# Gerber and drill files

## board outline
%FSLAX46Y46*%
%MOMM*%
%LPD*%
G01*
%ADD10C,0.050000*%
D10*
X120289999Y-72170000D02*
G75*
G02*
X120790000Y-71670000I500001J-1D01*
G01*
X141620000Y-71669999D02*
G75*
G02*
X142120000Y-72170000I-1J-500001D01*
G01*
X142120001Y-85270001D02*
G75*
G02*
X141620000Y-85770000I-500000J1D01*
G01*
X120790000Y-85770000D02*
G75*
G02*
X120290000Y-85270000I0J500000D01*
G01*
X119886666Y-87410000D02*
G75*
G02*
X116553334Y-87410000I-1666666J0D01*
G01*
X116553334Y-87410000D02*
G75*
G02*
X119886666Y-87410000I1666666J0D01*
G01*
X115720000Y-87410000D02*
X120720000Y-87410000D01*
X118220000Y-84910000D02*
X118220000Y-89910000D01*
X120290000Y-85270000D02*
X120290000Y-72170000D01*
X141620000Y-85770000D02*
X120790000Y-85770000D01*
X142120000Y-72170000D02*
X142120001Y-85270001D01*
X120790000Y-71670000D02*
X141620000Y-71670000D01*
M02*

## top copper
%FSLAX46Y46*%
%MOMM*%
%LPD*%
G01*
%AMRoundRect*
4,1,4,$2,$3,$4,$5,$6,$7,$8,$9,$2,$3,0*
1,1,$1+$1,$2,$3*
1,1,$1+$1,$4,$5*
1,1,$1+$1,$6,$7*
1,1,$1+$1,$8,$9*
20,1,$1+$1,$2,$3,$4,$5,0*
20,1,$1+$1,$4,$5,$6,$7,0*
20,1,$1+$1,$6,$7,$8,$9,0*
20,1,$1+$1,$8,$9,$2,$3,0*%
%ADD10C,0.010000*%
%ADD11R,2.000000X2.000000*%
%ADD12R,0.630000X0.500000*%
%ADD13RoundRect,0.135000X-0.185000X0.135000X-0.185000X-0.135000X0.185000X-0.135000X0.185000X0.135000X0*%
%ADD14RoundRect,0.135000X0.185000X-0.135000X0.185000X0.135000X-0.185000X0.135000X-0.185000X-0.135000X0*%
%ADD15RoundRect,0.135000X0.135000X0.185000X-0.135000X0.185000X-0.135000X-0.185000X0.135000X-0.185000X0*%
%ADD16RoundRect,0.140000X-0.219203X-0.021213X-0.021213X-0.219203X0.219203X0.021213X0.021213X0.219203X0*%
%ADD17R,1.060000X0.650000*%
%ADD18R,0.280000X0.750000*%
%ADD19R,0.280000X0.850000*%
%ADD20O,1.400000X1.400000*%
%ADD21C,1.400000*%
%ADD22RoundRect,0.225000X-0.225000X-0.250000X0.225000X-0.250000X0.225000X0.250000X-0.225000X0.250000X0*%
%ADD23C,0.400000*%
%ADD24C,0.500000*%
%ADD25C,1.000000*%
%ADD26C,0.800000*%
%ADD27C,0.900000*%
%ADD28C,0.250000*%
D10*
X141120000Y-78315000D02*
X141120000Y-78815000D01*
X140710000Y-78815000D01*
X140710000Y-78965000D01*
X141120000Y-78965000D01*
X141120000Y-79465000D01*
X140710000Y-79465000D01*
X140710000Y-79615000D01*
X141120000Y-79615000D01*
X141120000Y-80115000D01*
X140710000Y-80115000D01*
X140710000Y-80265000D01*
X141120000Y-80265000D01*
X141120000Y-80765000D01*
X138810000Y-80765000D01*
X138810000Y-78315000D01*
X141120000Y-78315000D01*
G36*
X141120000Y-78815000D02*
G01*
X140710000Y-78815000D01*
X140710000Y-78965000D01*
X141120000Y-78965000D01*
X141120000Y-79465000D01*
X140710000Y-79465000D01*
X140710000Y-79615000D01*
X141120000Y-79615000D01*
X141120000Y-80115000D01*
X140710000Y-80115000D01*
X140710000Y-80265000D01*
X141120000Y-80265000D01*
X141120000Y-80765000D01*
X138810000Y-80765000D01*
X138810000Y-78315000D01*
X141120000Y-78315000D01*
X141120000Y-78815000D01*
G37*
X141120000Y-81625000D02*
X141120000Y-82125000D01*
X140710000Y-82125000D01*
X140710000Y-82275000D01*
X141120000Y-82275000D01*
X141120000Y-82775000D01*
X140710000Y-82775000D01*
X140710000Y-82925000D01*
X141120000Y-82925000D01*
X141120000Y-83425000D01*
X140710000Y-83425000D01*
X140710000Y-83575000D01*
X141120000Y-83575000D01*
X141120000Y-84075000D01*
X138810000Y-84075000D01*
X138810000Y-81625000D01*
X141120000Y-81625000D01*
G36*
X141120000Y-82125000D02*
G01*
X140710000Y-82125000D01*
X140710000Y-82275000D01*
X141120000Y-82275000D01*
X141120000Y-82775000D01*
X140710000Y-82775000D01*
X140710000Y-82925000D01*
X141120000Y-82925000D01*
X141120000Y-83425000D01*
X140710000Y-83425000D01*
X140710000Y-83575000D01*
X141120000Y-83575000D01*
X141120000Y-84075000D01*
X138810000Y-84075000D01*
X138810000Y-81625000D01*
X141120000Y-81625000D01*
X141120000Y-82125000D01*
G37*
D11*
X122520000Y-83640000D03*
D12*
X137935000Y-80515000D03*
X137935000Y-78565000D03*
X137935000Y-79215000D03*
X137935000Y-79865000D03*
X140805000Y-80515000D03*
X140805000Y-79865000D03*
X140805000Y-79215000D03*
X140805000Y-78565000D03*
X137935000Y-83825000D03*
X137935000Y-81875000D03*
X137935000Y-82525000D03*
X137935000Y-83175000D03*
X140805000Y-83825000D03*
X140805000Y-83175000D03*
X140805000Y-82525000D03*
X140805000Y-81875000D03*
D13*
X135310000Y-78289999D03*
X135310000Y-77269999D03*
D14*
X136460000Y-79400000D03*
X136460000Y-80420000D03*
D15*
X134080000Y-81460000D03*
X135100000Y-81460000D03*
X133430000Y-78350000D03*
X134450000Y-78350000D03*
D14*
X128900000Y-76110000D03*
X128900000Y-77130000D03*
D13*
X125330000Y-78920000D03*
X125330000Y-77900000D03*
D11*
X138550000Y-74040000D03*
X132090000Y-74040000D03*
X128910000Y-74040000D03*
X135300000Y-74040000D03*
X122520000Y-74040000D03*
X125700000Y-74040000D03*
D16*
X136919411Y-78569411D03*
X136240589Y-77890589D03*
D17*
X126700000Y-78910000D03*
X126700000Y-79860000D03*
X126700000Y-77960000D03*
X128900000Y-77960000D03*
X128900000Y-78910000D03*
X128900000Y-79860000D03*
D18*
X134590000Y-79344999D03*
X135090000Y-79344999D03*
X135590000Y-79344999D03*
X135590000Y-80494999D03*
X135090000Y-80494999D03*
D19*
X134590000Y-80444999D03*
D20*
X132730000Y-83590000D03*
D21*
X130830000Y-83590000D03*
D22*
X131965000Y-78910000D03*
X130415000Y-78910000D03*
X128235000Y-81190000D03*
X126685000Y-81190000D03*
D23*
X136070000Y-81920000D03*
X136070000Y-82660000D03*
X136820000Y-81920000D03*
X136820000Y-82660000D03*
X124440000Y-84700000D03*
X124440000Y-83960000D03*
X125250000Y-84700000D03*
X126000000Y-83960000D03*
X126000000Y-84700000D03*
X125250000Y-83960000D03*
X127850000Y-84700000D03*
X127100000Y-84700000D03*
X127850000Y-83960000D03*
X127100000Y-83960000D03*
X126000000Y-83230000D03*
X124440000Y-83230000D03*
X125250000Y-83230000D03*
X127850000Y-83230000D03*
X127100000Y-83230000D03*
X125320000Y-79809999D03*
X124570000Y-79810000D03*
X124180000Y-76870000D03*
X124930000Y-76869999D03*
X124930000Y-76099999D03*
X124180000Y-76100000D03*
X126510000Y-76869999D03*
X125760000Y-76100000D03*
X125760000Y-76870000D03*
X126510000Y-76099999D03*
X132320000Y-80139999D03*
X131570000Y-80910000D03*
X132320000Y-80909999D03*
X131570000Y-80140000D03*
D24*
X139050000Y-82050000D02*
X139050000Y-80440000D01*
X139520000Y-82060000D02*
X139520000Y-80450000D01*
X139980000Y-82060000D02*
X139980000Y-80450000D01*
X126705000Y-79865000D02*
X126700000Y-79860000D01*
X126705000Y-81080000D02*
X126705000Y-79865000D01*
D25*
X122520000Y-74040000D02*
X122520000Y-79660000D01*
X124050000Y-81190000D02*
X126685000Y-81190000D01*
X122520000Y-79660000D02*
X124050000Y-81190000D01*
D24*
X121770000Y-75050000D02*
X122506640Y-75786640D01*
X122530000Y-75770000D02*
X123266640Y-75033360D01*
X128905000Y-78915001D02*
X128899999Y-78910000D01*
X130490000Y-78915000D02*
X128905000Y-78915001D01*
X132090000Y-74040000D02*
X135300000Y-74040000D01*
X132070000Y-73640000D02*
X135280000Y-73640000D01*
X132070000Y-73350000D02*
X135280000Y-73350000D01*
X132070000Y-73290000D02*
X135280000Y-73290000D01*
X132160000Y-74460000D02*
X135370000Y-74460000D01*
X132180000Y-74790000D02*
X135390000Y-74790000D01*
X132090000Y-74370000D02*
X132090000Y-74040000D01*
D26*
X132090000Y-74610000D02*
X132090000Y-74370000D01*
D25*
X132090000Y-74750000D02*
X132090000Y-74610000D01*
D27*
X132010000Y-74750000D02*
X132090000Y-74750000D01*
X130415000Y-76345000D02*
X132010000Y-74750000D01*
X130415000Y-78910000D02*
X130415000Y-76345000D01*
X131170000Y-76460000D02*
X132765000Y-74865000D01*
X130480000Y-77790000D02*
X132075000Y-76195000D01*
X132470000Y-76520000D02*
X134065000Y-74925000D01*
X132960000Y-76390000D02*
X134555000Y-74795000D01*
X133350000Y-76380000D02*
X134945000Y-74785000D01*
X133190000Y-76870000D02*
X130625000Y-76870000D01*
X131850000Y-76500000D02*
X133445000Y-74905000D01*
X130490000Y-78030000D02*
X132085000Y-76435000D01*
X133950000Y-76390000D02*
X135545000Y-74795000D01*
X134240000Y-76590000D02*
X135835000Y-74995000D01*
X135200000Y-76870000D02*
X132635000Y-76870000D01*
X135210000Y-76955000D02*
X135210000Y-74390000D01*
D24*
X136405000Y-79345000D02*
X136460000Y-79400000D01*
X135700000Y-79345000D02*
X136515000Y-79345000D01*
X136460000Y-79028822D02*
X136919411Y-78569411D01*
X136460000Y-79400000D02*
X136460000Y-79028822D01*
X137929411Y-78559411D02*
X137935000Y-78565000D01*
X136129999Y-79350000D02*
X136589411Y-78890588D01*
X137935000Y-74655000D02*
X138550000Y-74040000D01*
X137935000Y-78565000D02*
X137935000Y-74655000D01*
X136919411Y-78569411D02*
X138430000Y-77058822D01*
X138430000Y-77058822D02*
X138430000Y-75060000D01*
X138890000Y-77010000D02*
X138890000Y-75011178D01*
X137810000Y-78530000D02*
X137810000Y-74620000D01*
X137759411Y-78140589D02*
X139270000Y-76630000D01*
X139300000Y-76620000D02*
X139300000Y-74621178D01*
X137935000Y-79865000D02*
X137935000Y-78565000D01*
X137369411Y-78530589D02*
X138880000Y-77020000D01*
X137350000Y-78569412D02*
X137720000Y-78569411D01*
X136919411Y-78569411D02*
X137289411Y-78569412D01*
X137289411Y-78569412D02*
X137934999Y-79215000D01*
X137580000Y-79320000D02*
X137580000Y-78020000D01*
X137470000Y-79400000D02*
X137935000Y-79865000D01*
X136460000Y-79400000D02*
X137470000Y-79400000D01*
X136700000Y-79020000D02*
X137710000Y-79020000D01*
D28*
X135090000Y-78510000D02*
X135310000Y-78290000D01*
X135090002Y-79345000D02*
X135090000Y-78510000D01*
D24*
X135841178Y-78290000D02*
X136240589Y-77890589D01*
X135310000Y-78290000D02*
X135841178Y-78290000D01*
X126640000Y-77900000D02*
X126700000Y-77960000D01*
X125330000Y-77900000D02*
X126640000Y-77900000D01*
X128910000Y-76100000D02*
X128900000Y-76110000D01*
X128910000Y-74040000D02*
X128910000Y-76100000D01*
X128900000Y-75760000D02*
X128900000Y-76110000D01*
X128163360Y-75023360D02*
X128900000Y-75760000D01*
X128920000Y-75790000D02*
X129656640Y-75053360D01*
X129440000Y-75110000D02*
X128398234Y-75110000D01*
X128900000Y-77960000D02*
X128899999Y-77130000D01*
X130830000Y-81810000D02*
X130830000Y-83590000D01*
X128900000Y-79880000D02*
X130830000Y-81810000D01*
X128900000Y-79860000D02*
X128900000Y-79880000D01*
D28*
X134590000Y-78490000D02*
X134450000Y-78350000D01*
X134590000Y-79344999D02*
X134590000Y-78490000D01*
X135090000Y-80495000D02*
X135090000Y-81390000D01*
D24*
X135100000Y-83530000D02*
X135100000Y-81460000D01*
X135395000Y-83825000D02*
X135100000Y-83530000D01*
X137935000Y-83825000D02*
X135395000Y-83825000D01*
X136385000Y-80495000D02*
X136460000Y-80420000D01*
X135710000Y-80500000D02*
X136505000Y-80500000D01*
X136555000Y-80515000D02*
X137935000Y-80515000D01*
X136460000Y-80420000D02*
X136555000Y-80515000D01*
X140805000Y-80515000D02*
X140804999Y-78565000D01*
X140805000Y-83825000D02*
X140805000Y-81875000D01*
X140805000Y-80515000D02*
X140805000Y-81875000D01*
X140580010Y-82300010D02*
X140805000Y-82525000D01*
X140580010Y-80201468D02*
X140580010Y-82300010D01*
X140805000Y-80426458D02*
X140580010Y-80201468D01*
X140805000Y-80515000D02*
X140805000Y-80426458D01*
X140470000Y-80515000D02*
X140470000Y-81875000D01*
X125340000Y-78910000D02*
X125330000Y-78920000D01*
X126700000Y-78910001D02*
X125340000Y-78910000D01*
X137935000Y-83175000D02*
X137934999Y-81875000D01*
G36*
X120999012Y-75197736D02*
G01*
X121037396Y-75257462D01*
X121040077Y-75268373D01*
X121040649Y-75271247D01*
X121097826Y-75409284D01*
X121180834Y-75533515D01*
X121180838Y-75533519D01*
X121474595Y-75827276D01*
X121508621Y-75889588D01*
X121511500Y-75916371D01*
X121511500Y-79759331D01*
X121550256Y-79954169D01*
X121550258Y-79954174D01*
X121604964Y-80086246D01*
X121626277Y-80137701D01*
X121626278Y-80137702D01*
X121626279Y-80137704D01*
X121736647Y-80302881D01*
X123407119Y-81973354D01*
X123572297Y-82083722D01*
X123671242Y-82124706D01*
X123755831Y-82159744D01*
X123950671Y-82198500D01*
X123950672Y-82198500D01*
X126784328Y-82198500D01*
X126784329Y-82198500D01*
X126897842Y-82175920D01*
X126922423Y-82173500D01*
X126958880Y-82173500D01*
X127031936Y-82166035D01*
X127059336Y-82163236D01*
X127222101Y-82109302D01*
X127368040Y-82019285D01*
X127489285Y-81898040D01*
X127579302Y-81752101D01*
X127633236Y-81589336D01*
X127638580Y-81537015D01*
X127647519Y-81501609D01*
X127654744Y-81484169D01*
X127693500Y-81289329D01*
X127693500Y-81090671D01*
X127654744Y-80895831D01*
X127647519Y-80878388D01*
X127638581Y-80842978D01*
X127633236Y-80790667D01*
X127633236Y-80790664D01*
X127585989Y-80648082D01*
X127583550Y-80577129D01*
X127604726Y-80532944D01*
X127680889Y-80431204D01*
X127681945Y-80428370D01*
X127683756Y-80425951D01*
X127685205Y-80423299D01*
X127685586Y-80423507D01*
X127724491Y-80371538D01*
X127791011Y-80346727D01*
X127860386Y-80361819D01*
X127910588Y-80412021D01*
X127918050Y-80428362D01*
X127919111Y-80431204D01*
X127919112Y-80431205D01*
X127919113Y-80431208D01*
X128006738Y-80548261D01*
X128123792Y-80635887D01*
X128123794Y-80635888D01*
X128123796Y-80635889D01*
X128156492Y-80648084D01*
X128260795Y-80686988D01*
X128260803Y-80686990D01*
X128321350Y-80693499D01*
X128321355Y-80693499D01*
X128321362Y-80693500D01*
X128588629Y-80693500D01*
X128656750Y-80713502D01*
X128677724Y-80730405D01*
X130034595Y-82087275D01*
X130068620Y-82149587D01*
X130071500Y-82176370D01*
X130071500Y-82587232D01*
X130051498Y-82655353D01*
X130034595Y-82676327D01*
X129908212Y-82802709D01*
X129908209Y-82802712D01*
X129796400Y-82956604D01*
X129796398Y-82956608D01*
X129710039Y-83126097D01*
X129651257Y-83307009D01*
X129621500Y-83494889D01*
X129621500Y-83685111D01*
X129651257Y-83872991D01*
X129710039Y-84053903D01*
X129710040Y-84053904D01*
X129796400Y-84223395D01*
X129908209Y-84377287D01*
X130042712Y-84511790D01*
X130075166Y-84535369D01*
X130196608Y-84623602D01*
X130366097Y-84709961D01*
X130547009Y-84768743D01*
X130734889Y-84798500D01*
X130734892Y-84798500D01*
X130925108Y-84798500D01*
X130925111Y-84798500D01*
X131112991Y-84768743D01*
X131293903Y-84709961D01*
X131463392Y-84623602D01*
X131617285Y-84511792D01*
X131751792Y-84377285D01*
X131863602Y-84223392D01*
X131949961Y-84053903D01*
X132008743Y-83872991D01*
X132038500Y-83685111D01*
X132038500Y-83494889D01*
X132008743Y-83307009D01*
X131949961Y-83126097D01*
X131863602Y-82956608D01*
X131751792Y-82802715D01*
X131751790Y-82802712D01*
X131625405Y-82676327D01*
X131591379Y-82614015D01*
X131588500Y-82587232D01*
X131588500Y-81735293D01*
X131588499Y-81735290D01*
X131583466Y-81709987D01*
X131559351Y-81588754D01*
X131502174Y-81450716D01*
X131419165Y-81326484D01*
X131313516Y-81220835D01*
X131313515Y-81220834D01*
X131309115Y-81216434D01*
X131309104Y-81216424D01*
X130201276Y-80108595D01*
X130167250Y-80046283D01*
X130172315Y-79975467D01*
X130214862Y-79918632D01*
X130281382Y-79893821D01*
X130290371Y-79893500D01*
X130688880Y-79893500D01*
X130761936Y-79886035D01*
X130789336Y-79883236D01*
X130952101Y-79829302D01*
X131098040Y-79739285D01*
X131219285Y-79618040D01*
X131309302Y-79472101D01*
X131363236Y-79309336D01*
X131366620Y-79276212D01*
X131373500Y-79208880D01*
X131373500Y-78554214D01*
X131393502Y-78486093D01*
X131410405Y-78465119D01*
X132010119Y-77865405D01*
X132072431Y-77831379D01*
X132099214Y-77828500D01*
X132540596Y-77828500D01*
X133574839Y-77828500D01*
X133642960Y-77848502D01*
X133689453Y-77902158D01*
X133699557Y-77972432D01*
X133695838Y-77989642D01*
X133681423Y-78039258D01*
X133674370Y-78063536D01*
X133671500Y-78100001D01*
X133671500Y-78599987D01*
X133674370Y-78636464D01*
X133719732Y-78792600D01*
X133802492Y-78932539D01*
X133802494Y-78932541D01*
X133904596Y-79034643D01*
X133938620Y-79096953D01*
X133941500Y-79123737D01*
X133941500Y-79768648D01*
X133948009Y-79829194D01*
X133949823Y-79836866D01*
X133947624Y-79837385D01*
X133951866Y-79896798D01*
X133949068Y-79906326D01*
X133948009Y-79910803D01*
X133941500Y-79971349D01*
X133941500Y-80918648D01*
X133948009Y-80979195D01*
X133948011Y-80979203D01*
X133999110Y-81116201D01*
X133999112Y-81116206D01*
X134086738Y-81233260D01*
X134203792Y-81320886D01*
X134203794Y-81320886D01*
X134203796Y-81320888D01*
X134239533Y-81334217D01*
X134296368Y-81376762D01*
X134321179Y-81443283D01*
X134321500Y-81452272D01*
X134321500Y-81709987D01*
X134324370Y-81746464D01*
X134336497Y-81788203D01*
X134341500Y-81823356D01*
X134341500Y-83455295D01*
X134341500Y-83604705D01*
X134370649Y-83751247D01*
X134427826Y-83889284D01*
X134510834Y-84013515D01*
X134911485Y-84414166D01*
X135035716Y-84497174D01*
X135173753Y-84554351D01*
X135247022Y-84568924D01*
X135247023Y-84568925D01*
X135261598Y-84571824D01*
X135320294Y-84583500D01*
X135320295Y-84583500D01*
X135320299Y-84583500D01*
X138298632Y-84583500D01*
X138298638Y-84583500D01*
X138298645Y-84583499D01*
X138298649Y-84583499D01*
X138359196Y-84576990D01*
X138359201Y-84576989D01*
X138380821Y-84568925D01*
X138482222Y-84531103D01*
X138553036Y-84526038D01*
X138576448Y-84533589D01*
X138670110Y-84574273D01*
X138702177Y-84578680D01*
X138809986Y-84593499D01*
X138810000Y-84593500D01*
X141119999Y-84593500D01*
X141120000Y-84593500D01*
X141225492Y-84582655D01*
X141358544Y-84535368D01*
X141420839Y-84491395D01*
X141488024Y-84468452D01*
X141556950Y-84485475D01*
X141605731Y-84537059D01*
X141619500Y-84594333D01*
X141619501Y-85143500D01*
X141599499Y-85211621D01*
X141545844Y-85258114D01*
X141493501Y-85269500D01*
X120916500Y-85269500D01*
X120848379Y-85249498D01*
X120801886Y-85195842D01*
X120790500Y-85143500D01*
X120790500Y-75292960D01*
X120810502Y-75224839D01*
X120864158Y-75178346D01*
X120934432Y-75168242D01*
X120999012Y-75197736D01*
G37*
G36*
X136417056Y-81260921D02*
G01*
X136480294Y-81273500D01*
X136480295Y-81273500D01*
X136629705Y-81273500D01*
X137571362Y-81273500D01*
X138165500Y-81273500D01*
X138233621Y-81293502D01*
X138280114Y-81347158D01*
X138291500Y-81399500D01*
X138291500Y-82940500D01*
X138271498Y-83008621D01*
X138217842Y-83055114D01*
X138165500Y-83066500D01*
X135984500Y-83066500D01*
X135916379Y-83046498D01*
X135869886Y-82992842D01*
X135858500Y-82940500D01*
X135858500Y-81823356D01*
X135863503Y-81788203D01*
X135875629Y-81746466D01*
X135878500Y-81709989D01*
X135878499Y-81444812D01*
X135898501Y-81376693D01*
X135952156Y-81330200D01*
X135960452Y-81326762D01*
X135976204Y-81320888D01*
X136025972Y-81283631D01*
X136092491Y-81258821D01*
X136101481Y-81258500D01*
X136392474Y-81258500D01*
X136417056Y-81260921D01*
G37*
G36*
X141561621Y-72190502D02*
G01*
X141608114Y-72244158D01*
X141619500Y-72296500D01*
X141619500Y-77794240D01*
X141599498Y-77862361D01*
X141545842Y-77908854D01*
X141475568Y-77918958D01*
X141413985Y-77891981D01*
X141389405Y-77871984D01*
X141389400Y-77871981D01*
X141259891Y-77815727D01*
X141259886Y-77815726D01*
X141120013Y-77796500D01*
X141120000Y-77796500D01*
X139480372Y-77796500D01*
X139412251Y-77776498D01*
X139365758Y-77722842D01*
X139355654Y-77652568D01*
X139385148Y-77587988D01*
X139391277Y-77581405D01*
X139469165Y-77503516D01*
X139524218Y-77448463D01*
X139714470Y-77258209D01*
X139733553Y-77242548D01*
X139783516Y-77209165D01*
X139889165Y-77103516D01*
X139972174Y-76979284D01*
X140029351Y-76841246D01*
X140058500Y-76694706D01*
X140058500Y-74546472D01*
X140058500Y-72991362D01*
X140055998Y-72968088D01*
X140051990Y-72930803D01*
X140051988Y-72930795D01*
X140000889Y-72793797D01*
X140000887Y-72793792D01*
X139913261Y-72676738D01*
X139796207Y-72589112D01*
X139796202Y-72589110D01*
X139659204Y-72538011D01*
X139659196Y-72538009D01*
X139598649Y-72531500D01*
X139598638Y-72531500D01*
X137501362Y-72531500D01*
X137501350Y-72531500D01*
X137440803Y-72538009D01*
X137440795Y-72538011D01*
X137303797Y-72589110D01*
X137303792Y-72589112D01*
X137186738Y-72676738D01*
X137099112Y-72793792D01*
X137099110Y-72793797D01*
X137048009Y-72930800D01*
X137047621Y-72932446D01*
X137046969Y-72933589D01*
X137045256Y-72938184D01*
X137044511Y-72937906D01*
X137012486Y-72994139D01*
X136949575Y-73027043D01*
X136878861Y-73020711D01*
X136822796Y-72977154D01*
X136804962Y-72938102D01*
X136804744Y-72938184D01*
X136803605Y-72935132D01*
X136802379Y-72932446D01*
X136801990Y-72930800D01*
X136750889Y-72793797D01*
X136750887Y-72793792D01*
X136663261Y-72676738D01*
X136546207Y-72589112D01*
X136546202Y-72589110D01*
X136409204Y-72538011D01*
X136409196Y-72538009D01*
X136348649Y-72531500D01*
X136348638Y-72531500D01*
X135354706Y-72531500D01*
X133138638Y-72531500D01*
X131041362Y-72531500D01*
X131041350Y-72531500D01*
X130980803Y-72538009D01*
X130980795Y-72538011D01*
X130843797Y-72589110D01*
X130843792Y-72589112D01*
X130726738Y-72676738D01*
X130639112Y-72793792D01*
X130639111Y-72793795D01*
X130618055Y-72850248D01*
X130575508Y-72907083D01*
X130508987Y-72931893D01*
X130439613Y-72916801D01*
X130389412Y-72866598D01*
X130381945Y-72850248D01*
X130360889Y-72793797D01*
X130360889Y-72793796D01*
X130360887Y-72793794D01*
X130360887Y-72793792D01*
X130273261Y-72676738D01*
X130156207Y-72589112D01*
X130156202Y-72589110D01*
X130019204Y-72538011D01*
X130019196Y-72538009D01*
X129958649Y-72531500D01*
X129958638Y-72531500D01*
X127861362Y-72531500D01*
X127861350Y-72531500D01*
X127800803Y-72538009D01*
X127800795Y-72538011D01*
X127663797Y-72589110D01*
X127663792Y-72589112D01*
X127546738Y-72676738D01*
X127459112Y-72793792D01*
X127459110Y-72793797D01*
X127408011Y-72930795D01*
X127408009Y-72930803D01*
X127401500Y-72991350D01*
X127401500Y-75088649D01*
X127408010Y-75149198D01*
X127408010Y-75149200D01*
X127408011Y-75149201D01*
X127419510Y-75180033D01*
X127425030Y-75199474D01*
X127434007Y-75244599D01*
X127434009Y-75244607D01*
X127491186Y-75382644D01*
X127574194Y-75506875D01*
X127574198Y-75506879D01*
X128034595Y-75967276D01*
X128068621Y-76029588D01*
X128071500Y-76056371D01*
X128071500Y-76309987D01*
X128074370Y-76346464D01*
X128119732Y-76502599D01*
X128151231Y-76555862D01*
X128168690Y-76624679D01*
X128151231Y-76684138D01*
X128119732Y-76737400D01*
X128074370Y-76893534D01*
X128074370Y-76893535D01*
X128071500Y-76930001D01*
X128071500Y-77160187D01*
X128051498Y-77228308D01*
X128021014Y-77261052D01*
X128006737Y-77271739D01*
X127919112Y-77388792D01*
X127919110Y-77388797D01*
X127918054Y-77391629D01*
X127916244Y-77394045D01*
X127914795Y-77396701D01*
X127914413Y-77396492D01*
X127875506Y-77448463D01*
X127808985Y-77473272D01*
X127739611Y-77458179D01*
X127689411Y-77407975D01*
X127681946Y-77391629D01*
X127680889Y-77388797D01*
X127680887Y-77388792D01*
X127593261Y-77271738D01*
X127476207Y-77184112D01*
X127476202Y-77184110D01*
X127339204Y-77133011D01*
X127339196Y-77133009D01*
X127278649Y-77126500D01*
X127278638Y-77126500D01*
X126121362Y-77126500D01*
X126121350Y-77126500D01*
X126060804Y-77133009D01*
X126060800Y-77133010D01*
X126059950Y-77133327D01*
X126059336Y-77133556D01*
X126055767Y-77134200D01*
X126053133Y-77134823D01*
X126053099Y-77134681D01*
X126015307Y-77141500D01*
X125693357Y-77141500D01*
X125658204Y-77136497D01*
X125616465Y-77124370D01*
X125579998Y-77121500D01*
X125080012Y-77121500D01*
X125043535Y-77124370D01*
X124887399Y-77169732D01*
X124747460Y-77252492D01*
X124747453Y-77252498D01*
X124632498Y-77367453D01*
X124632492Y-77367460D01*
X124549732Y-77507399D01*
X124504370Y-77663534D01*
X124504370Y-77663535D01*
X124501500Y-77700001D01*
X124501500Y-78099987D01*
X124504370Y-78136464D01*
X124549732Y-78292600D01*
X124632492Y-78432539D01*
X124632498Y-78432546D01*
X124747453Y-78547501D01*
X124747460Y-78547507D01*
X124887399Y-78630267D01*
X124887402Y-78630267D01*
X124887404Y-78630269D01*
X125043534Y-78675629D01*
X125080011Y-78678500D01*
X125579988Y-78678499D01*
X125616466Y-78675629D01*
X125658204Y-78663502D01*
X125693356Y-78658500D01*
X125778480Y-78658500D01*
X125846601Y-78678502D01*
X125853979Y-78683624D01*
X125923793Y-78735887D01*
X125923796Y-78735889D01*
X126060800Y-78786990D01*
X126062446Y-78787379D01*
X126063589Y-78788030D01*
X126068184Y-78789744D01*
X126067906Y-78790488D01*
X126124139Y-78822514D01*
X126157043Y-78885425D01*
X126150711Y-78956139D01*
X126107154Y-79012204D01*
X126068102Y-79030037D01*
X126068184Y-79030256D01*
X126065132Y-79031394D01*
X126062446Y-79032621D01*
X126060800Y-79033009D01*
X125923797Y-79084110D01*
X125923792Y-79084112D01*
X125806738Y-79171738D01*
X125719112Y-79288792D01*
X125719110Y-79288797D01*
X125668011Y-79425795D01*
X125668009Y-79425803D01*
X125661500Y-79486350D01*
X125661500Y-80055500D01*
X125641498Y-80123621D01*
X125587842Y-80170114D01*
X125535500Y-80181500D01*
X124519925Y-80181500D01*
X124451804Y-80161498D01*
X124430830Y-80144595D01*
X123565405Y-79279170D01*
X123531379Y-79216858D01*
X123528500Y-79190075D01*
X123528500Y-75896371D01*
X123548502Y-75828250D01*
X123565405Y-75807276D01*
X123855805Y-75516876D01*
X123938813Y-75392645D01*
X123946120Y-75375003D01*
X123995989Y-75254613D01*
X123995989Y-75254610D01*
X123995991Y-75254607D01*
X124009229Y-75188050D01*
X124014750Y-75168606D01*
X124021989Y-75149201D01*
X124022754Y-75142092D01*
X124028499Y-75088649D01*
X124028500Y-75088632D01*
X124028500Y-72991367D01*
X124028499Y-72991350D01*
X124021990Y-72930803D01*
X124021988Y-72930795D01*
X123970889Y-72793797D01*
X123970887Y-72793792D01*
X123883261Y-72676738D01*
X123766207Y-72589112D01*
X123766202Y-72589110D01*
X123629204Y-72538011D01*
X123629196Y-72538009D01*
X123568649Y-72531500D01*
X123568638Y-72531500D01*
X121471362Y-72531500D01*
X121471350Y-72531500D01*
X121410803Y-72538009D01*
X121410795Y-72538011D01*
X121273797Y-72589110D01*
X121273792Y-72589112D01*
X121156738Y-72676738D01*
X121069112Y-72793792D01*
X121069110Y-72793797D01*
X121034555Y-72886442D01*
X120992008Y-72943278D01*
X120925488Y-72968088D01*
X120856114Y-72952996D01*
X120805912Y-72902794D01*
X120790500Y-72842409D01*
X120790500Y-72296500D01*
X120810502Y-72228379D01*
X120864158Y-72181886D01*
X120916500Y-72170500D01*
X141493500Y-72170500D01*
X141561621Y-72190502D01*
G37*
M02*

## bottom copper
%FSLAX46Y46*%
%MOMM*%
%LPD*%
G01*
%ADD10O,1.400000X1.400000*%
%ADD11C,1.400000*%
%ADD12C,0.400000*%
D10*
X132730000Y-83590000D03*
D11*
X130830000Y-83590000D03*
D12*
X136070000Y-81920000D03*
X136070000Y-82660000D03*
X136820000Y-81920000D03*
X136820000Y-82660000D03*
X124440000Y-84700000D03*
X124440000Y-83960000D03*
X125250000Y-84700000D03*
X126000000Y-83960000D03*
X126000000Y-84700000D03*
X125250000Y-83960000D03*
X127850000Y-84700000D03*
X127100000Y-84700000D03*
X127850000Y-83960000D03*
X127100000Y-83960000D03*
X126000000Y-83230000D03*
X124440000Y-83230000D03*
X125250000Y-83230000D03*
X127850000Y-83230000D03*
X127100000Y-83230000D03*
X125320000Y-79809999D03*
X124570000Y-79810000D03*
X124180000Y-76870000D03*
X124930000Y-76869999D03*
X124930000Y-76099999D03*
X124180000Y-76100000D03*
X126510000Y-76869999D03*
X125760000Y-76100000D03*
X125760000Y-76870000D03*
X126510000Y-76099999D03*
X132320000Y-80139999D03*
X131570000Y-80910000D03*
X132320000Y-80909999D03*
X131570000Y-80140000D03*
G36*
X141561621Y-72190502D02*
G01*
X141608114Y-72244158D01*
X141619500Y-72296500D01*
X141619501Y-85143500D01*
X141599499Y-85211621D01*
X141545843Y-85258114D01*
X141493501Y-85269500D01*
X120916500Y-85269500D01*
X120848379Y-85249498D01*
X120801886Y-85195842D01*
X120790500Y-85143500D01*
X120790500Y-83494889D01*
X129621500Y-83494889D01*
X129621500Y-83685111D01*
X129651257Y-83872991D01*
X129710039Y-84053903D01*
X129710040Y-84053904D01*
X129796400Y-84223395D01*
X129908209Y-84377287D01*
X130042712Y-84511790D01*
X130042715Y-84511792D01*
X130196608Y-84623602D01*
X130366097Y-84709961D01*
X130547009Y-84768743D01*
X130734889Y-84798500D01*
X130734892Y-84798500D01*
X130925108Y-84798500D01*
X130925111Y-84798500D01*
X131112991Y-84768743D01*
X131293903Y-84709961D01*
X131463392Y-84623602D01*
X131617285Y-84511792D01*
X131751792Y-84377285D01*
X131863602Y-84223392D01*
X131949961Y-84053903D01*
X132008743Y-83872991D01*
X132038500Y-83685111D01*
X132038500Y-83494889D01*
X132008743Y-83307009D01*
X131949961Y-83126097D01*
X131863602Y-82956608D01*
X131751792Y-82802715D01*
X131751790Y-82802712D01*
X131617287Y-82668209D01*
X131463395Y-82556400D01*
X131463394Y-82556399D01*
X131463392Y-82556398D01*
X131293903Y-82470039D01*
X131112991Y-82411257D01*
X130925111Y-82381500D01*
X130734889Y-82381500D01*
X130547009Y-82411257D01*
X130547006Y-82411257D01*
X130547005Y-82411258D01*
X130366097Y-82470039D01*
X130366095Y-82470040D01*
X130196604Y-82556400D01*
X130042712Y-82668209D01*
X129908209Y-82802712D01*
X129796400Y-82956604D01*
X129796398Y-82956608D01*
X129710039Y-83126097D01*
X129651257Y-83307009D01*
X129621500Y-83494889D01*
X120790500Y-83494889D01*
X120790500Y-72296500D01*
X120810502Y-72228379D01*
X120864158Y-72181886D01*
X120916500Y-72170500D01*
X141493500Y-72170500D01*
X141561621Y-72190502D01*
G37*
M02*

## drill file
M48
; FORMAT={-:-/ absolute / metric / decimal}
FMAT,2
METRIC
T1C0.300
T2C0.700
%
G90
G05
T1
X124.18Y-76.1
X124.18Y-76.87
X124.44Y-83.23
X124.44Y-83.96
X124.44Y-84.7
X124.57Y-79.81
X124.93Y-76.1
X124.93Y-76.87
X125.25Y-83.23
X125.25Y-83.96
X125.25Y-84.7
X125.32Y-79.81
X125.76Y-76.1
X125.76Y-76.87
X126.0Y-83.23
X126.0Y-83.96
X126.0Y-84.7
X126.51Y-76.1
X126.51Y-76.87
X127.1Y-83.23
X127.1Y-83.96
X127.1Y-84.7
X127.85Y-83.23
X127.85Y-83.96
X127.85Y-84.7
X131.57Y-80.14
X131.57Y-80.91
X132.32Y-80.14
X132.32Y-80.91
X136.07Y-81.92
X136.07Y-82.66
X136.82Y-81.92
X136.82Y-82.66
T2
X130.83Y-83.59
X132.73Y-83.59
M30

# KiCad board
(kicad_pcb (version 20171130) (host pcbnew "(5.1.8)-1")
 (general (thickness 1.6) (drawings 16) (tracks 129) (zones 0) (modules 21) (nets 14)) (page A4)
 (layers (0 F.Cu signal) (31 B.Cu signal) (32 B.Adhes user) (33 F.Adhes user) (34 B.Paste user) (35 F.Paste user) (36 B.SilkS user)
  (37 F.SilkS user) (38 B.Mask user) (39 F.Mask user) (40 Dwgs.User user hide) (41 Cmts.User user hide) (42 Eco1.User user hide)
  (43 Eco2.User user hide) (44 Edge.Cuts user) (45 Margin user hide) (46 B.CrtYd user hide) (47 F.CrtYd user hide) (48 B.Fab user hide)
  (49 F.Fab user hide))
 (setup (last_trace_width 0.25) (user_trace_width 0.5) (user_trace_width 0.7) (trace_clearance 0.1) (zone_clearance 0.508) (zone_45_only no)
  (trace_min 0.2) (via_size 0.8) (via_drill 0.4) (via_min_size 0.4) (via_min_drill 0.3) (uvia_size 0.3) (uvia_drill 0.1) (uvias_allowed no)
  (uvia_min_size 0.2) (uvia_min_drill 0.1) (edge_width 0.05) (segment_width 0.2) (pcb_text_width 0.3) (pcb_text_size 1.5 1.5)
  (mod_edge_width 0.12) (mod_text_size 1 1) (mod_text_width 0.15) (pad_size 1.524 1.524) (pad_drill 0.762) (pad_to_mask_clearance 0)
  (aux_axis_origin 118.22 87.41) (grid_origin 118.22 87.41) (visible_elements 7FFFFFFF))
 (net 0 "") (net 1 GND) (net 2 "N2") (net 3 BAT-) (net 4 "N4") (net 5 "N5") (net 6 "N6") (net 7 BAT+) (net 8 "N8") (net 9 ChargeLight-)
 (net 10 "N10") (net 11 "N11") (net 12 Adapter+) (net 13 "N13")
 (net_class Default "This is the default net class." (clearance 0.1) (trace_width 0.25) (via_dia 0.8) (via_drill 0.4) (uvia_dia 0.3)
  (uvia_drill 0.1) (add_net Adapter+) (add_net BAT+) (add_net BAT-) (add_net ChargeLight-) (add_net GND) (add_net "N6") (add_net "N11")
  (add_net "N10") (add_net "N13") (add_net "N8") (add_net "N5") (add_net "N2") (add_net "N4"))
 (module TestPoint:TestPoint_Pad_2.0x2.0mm (layer F.Cu) (at 122.52 83.64)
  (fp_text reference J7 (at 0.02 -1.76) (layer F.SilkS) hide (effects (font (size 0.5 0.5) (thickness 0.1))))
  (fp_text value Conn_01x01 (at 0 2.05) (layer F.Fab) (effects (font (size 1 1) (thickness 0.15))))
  (pad 1 smd rect (at 0 0) (size 2 2) (layers F.Cu F.Mask) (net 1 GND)))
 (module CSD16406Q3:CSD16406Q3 (layer F.Cu) (at 139.37 79.54)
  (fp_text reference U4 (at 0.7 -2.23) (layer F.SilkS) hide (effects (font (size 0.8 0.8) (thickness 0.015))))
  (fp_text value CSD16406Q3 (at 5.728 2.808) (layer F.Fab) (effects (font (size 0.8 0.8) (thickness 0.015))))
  (fp_poly
   (pts (xy 1.75 -1.225) (xy 1.75 -0.725) (xy 1.34 -0.725) (xy 1.34 -0.575) (xy 1.75 -0.575) (xy 1.75 -0.075) (xy 1.34 -0.075)
    (xy 1.34 0.075) (xy 1.75 0.075) (xy 1.75 0.575) (xy 1.34 0.575) (xy 1.34 0.725) (xy 1.75 0.725) (xy 1.75 1.225) (xy -0.56 1.225)
    (xy -0.56 -1.225))
   (layer F.Cu) (width 0.01))
  (pad 4 smd rect (at -1.435 0.975) (size 0.63 0.5) (layers F.Cu F.Mask) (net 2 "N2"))
  (pad 1 smd rect (at -1.435 -0.975) (size 0.63 0.5) (layers F.Cu F.Mask) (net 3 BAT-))
  (pad 2 smd rect (at -1.435 -0.325) (size 0.63 0.5) (layers F.Cu F.Mask) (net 3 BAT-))
  (pad 3 smd rect (at -1.435 0.325) (size 0.63 0.5) (layers F.Cu F.Mask) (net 3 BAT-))
  (pad 5 smd rect (at 1.435 0.975) (size 0.63 0.5) (layers F.Cu) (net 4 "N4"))
  (pad 6 smd rect (at 1.435 0.325) (size 0.63 0.5) (layers F.Cu) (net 4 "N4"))
  (pad 7 smd rect (at 1.435 -0.325) (size 0.63 0.5) (layers F.Cu) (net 4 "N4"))
  (pad 8 smd rect (at 1.435 -0.975) (size 0.63 0.5) (layers F.Cu) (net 4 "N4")))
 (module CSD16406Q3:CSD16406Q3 (layer F.Cu) (at 139.37 82.85)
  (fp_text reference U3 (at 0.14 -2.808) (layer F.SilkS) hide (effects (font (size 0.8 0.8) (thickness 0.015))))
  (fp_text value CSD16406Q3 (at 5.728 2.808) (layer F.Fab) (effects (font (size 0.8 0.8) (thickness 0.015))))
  (fp_poly
   (pts (xy 1.75 -1.225) (xy 1.75 -0.725) (xy 1.34 -0.725) (xy 1.34 -0.575) (xy 1.75 -0.575) (xy 1.75 -0.075) (xy 1.34 -0.075)
    (xy 1.34 0.075) (xy 1.75 0.075) (xy 1.75 0.575) (xy 1.34 0.575) (xy 1.34 0.725) (xy 1.75 0.725) (xy 1.75 1.225) (xy -0.56 1.225)
    (xy -0.56 -1.225))
   (layer F.Cu) (width 0.01))
  (pad 4 smd rect (at -1.435 0.975) (size 0.63 0.5) (layers F.Cu F.Mask) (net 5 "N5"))
  (pad 1 smd rect (at -1.435 -0.975) (size 0.63 0.5) (layers F.Cu F.Mask) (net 1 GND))
  (pad 2 smd rect (at -1.435 -0.325) (size 0.63 0.5) (layers F.Cu F.Mask) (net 1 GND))
  (pad 3 smd rect (at -1.435 0.325) (size 0.63 0.5) (layers F.Cu F.Mask) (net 1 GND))
  (pad 5 smd rect (at 1.435 0.975) (size 0.63 0.5) (layers F.Cu) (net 4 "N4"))
  (pad 6 smd rect (at 1.435 0.325) (size 0.63 0.5) (layers F.Cu) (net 4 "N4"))
  (pad 7 smd rect (at 1.435 -0.325) (size 0.63 0.5) (layers F.Cu) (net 4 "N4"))
  (pad 8 smd rect (at 1.435 -0.975) (size 0.63 0.5) (layers F.Cu) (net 4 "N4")))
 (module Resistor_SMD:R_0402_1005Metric (layer F.Cu) (at 135.31 77.779999 270)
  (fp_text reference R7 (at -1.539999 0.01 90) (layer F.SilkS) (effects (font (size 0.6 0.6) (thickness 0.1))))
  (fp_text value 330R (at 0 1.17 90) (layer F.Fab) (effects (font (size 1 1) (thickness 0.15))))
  (pad 2 smd roundrect (at 0.51 0 270) (size 0.54 0.64) (layers F.Cu F.Paste F.Mask) (roundrect_rratio 0.25) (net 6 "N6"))
  (pad 1 smd roundrect (at -0.51 0 270) (size 0.54 0.64) (layers F.Cu F.Paste F.Mask) (roundrect_rratio 0.25) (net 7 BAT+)))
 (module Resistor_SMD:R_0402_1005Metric (layer F.Cu) (at 136.46 79.91 90)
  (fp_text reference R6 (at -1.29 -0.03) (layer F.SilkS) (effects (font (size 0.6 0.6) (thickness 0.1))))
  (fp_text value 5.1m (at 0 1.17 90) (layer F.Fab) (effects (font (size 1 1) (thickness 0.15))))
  (pad 2 smd roundrect (at 0.51 0 90) (size 0.54 0.64) (layers F.Cu F.Paste F.Mask) (roundrect_rratio 0.25) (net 3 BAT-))
  (pad 1 smd roundrect (at -0.51 0 90) (size 0.54 0.64) (layers F.Cu F.Paste F.Mask) (roundrect_rratio 0.25) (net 2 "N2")))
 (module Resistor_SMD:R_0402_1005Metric (layer F.Cu) (at 134.59 81.46 180)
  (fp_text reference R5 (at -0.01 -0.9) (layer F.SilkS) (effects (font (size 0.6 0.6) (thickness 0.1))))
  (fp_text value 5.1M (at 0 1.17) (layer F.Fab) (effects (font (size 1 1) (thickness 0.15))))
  (pad 2 smd roundrect (at 0.51 0 180) (size 0.54 0.64) (layers F.Cu F.Paste F.Mask) (roundrect_rratio 0.25) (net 1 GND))
  (pad 1 smd roundrect (at -0.51 0 180) (size 0.54 0.64) (layers F.Cu F.Paste F.Mask) (roundrect_rratio 0.25) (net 5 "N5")))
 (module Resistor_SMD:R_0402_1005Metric (layer F.Cu) (at 133.94 78.35 180)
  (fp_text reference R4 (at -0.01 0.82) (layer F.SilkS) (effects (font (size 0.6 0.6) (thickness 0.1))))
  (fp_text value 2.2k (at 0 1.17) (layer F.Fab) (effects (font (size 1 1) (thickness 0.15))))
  (pad 2 smd roundrect (at 0.51 0 180) (size 0.54 0.64) (layers F.Cu F.Paste F.Mask) (roundrect_rratio 0.25) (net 1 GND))
  (pad 1 smd roundrect (at -0.51 0 180) (size 0.54 0.64) (layers F.Cu F.Paste F.Mask) (roundrect_rratio 0.25) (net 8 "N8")))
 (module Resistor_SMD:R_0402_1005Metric (layer F.Cu) (at 128.9 76.62 90)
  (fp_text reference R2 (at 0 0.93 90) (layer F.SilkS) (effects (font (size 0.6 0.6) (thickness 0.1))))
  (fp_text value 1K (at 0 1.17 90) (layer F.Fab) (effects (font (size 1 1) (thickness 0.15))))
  (pad 2 smd roundrect (at 0.51 0 90) (size 0.54 0.64) (layers F.Cu F.Paste F.Mask) (roundrect_rratio 0.25) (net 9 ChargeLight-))
  (pad 1 smd roundrect (at -0.51 0 90) (size 0.54 0.64) (layers F.Cu F.Paste F.Mask) (roundrect_rratio 0.25) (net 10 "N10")))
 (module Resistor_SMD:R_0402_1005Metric (layer F.Cu) (at 125.33 78.41 270)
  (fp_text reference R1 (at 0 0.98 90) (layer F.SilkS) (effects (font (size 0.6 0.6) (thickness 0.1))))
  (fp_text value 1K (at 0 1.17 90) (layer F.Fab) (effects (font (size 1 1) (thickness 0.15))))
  (pad 2 smd roundrect (at 0.51 0 270) (size 0.54 0.64) (layers F.Cu F.Paste F.Mask) (roundrect_rratio 0.25) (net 1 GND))
  (pad 1 smd roundrect (at -0.51 0 270) (size 0.54 0.64) (layers F.Cu F.Paste F.Mask) (roundrect_rratio 0.25) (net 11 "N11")))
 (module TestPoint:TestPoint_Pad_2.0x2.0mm (layer F.Cu) (at 138.55 74.04 180)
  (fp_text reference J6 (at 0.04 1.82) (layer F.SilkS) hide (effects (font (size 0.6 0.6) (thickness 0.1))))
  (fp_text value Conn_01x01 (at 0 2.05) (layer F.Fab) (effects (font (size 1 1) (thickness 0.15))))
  (pad 1 smd rect (at 0 0 180) (size 2 2) (layers F.Cu F.Mask) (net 3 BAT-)))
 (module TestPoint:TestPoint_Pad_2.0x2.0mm (layer F.Cu) (at 132.09 74.04 180)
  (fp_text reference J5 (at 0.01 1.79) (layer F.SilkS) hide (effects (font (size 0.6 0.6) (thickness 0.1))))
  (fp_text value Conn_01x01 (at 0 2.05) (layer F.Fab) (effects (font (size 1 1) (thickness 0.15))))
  (pad 1 smd rect (at 0 0 180) (size 2 2) (layers F.Cu F.Mask) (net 7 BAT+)))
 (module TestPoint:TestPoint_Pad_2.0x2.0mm (layer F.Cu) (at 128.91 74.04 180)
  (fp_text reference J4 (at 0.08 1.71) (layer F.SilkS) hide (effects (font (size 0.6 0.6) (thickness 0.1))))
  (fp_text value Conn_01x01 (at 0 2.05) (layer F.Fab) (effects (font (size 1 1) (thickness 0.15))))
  (pad 1 smd rect (at 0 0 180) (size 2 2) (layers F.Cu F.Mask) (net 9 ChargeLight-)))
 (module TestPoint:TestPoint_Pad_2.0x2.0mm (layer F.Cu) (at 135.3 74.04 180)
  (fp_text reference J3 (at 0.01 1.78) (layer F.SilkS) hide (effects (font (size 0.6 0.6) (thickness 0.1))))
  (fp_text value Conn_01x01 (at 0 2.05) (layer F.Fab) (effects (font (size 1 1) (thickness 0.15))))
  (pad 1 smd rect (at 0 0 180) (size 2 2) (layers F.Cu F.Mask) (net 7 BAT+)))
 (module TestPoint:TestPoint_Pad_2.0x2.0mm (layer F.Cu) (at 122.52 74.04 180)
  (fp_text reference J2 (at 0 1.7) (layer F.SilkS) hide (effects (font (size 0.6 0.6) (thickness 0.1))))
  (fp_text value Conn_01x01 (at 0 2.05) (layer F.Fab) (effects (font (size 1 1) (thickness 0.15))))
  (pad 1 smd rect (at 0 0 180) (size 2 2) (layers F.Cu F.Mask) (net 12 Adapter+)))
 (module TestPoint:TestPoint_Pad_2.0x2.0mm (layer F.Cu) (at 125.7 74.04 180)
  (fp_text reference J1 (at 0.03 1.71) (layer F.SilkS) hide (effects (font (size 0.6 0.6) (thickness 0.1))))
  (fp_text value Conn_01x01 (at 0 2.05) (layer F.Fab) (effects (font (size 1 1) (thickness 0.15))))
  (pad 1 smd rect (at 0 0 180) (size 2 2) (layers F.Cu F.Mask) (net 1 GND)))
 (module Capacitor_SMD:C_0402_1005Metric (layer F.Cu) (at 136.58 78.23 315)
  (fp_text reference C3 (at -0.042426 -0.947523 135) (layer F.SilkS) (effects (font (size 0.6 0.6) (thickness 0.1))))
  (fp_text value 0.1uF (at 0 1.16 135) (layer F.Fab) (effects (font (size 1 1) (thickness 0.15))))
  (pad 2 smd roundrect (at 0.48 0 315) (size 0.56 0.62) (layers F.Cu F.Paste F.Mask) (roundrect_rratio 0.25) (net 3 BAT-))
  (pad 1 smd roundrect (at -0.48 0 315) (size 0.56 0.62) (layers F.Cu F.Paste F.Mask) (roundrect_rratio 0.25) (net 6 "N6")))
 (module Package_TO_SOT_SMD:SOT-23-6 (layer F.Cu) (at 127.8 78.91 180)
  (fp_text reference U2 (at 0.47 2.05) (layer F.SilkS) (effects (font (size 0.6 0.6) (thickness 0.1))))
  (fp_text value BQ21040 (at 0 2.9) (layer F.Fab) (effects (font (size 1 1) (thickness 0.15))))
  (pad 5 smd rect (at 1.1 0 180) (size 1.06 0.65) (layers F.Cu F.Paste F.Mask) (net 1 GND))
  (pad 6 smd rect (at 1.1 -0.95 180) (size 1.06 0.65) (layers F.Cu F.Paste F.Mask) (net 12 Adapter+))
  (pad 4 smd rect (at 1.1 0.95 180) (size 1.06 0.65) (layers F.Cu F.Paste F.Mask) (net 11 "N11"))
  (pad 3 smd rect (at -1.1 0.95 180) (size 1.06 0.65) (layers F.Cu F.Paste F.Mask) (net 10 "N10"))
  (pad 2 smd rect (at -1.1 0 180) (size 1.06 0.65) (layers F.Cu F.Paste F.Mask) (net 7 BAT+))
  (pad 1 smd rect (at -1.1 -0.95 180) (size 1.06 0.65) (layers F.Cu F.Paste F.Mask) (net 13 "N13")))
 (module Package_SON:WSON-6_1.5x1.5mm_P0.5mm (layer F.Cu) (at 135.09 79.919999 90)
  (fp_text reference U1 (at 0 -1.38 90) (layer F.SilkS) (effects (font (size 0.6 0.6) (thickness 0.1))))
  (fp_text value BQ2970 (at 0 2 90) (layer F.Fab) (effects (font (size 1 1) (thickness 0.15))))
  (pad 6 smd rect (at 0.575 -0.5) (size 0.28 0.75) (layers F.Cu F.Paste F.Mask) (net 8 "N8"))
  (pad 5 smd rect (at 0.575 0) (size 0.28 0.75) (layers F.Cu F.Paste F.Mask) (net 6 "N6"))
  (pad 4 smd rect (at 0.575 0.5) (size 0.28 0.75) (layers F.Cu F.Paste F.Mask) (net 3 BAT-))
  (pad 3 smd rect (at -0.575 0.5) (size 0.28 0.75) (layers F.Cu F.Paste F.Mask) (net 2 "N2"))
  (pad 2 smd rect (at -0.575 0) (size 0.28 0.75) (layers F.Cu F.Paste F.Mask) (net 5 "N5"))
  (pad 1 smd rect (at -0.525 -0.5) (size 0.28 0.85) (layers F.Cu F.Paste F.Mask)))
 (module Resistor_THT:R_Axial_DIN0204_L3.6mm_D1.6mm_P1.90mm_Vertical (layer F.Cu) (at 130.83 83.59)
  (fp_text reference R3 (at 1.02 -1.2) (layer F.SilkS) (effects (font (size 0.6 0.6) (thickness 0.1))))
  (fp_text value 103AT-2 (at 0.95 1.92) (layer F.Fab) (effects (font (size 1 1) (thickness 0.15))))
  (pad 2 thru_hole oval (at 1.9 0) (size 1.4 1.4) (drill 0.7) (layers *.Cu *.Mask) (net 1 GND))
  (pad 1 thru_hole circle (at 0 0) (size 1.4 1.4) (drill 0.7) (layers *.Cu *.Mask) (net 13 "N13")))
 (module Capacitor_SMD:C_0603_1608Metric (layer F.Cu) (at 131.19 78.91)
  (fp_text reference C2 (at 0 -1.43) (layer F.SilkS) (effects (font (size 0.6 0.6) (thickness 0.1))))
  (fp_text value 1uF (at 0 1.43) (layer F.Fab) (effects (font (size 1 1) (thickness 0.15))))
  (pad 2 smd roundrect (at 0.775 0) (size 0.9 0.95) (layers F.Cu F.Paste F.Mask) (roundrect_rratio 0.25) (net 1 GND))
  (pad 1 smd roundrect (at -0.775 0) (size 0.9 0.95) (layers F.Cu F.Paste F.Mask) (roundrect_rratio 0.25) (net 7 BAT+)))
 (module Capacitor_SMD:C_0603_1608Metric (layer F.Cu) (at 127.46 81.19)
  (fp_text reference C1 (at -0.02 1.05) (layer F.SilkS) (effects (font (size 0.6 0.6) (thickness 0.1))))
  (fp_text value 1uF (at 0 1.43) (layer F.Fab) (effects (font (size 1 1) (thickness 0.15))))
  (pad 2 smd roundrect (at 0.775 0) (size 0.9 0.95) (layers F.Cu F.Paste F.Mask) (roundrect_rratio 0.25) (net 1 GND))
  (pad 1 smd roundrect (at -0.775 0) (size 0.9 0.95) (layers F.Cu F.Paste F.Mask) (roundrect_rratio 0.25) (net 12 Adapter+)))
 (gr_arc (start 120.79 72.170001) (end 120.79 71.67) (angle -89.99988541) (layer Edge.Cuts) (width 0.05))
 (gr_arc (start 141.619999 72.17) (end 142.12 72.17) (angle -89.99988541) (layer Edge.Cuts) (width 0.05))
 (gr_arc (start 141.620001 85.27) (end 141.62 85.77) (angle -90) (layer Edge.Cuts) (width 0.05))
 (gr_arc (start 120.79 85.27) (end 120.29 85.27) (angle -90) (layer Edge.Cuts) (width 0.05))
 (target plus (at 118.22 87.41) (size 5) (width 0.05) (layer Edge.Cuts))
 (gr_line (start 120.29 85.27) (end 120.29 72.17) (layer Edge.Cuts) (width 0.05))
 (gr_line (start 141.62 85.77) (end 120.79 85.77) (layer Edge.Cuts) (width 0.05))
 (gr_line (start 142.12 72.17) (end 142.120001 85.270001) (layer Edge.Cuts) (width 0.05))
 (gr_line (start 120.79 71.67) (end 141.62 71.67) (layer Edge.Cuts) (width 0.05))
 (segment (start 139.05 82.05) (end 139.05 80.44) (width 0.5) (layer F.Cu) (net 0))
 (segment (start 139.52 82.06) (end 139.52 80.45) (width 0.5) (layer F.Cu) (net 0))
 (segment (start 139.98 82.06) (end 139.98 80.45) (width 0.5) (layer F.Cu) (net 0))
 (segment (start 126.705 79.865) (end 126.7 79.86) (width 0.5) (layer F.Cu) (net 12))
 (segment (start 126.705 81.08) (end 126.705 79.865) (width 0.5) (layer F.Cu) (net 12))
 (segment (start 122.52 74.04) (end 122.52 79.66) (width 1) (layer F.Cu) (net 12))
 (segment (start 124.05 81.19) (end 126.685 81.19) (width 1) (layer F.Cu) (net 12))
 (segment (start 122.52 79.66) (end 124.05 81.19) (width 1) (layer F.Cu) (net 12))
 (segment (start 121.77 75.05) (end 122.50664 75.78664) (width 0.5) (layer F.Cu) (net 12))
 (segment (start 122.53 75.77) (end 123.26664 75.03336) (width 0.5) (layer F.Cu) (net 12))
 (segment (start 128.905 78.915001) (end 128.899999 78.91) (width 0.5) (layer F.Cu) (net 7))
 (segment (start 130.49 78.915) (end 128.905 78.915001) (width 0.5) (layer F.Cu) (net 7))
 (segment (start 132.09 74.04) (end 135.3 74.04) (width 0.5) (layer F.Cu) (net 7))
 (segment (start 132.07 73.64) (end 135.28 73.64) (width 0.5) (layer F.Cu) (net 7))
 (segment (start 132.07 73.35) (end 135.28 73.35) (width 0.5) (layer F.Cu) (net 7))
 (segment (start 132.07 73.29) (end 135.28 73.29) (width 0.5) (layer F.Cu) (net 7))
 (segment (start 132.16 74.46) (end 135.37 74.46) (width 0.5) (layer F.Cu) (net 7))
 (segment (start 132.18 74.79) (end 135.39 74.79) (width 0.5) (layer F.Cu) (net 7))
 (segment (start 132.09 74.37) (end 132.09 74.04) (width 0.5) (layer F.Cu) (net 7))
 (segment (start 132.09 74.61) (end 132.09 74.37) (width 0.8) (layer F.Cu) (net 7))
 (segment (start 132.09 74.75) (end 132.09 74.61) (width 1) (layer F.Cu) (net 7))
 (segment (start 132.01 74.75) (end 132.09 74.75) (width 0.9) (layer F.Cu) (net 7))
 (segment (start 130.415 76.345) (end 132.01 74.75) (width 0.9) (layer F.Cu) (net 7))
 (segment (start 130.415 78.91) (end 130.415 76.345) (width 0.9) (layer F.Cu) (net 7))
 (segment (start 131.17 76.46) (end 132.765 74.865) (width 0.9) (layer F.Cu) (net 7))
 (segment (start 130.48 77.79) (end 132.075 76.195) (width 0.9) (layer F.Cu) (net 7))
 (segment (start 132.47 76.52) (end 134.065 74.925) (width 0.9) (layer F.Cu) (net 7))
 (segment (start 132.96 76.39) (end 134.555 74.795) (width 0.9) (layer F.Cu) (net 7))
 (segment (start 133.35 76.38) (end 134.945 74.785) (width 0.9) (layer F.Cu) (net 7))
 (segment (start 133.19 76.87) (end 130.625 76.87) (width 0.9) (layer F.Cu) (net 7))
 (segment (start 131.85 76.5) (end 133.445 74.905) (width 0.9) (layer F.Cu) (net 7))
 (segment (start 130.49 78.03) (end 132.085 76.435) (width 0.9) (layer F.Cu) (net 7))
 (segment (start 133.95 76.39) (end 135.545 74.795) (width 0.9) (layer F.Cu) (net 7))
 (segment (start 134.24 76.59) (end 135.835 74.995) (width 0.9) (layer F.Cu) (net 7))
 (segment (start 135.2 76.87) (end 132.635 76.87) (width 0.9) (layer F.Cu) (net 7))
 (segment (start 135.21 76.955) (end 135.21 74.39) (width 0.9) (layer F.Cu) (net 7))
 (segment (start 136.405 79.345) (end 136.46 79.4) (width 0.5) (layer F.Cu) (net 3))
 (segment (start 135.7 79.345) (end 136.515 79.345) (width 0.5) (layer F.Cu) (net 3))
 (segment (start 136.46 79.028822) (end 136.919411 78.569411) (width 0.5) (layer F.Cu) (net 3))
 (segment (start 136.46 79.4) (end 136.46 79.028822) (width 0.5) (layer F.Cu) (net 3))
 (segment (start 137.929411 78.559411) (end 137.935 78.565) (width 0.5) (layer F.Cu) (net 3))
 (segment (start 136.129999 79.35) (end 136.589411 78.890588) (width 0.5) (layer F.Cu) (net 3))
 (segment (start 137.935 74.655) (end 138.55 74.04) (width 0.5) (layer F.Cu) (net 3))
 (segment (start 137.935 78.565) (end 137.935 74.655) (width 0.5) (layer F.Cu) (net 3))
 (segment (start 136.919411 78.569411) (end 138.43 77.058822) (width 0.5) (layer F.Cu) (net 3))
 (segment (start 138.43 77.058822) (end 138.43 75.06) (width 0.5) (layer F.Cu) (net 3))
 (segment (start 138.89 77.01) (end 138.89 75.011178) (width 0.5) (layer F.Cu) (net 3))
 (segment (start 137.81 78.53) (end 137.81 74.62) (width 0.5) (layer F.Cu) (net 3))
 (segment (start 137.759411 78.140589) (end 139.27 76.63) (width 0.5) (layer F.Cu) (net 3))
 (segment (start 139.3 76.62) (end 139.3 74.621178) (width 0.5) (layer F.Cu) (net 3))
 (segment (start 137.935 79.865) (end 137.935 78.565) (width 0.5) (layer F.Cu) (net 3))
 (segment (start 137.369411 78.530589) (end 138.88 77.02) (width 0.5) (layer F.Cu) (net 3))
 (segment (start 137.35 78.569412) (end 137.72 78.569411) (width 0.5) (layer F.Cu) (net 3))
 (segment (start 136.919411 78.569411) (end 137.289411 78.569412) (width 0.5) (layer F.Cu) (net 3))
 (segment (start 137.289411 78.569412) (end 137.934999 79.215) (width 0.5) (layer F.Cu) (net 3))
 (segment (start 137.58 79.32) (end 137.58 78.02) (width 0.5) (layer F.Cu) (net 3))
 (segment (start 137.47 79.4) (end 137.935 79.865) (width 0.5) (layer F.Cu) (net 3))
 (segment (start 136.46 79.4) (end 137.47 79.4) (width 0.5) (layer F.Cu) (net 3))
 (segment (start 136.7 79.02) (end 137.71 79.02) (width 0.5) (layer F.Cu) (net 3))
 (segment (start 135.09 78.51) (end 135.31 78.29) (width 0.25) (layer F.Cu) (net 6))
 (segment (start 135.090002 79.345) (end 135.09 78.51) (width 0.25) (layer F.Cu) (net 6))
 (segment (start 135.841178 78.29) (end 136.240589 77.890589) (width 0.5) (layer F.Cu) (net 6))
 (segment (start 135.31 78.29) (end 135.841178 78.29) (width 0.5) (layer F.Cu) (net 6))
 (segment (start 126.64 77.9) (end 126.7 77.96) (width 0.5) (layer F.Cu) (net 11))
 (segment (start 125.33 77.9) (end 126.64 77.9) (width 0.5) (layer F.Cu) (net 11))
 (segment (start 128.91 76.1) (end 128.9 76.11) (width 0.5) (layer F.Cu) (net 9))
 (segment (start 128.91 74.04) (end 128.91 76.1) (width 0.5) (layer F.Cu) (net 9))
 (segment (start 128.9 75.76) (end 128.9 76.11) (width 0.5) (layer F.Cu) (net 9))
 (segment (start 128.16336 75.02336) (end 128.9 75.76) (width 0.5) (layer F.Cu) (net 9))
 (segment (start 128.92 75.79) (end 129.65664 75.05336) (width 0.5) (layer F.Cu) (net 9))
 (segment (start 129.44 75.11) (end 128.398234 75.11) (width 0.5) (layer F.Cu) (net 9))
 (segment (start 128.9 77.96) (end 128.899999 77.13) (width 0.5) (layer F.Cu) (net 10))
 (segment (start 130.83 81.81) (end 130.83 83.59) (width 0.5) (layer F.Cu) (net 13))
 (segment (start 128.9 79.88) (end 130.83 81.81) (width 0.5) (layer F.Cu) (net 13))
 (segment (start 128.9 79.86) (end 128.9 79.88) (width 0.5) (layer F.Cu) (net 13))
 (segment (start 134.59 78.49) (end 134.45 78.35) (width 0.25) (layer F.Cu) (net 8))
 (segment (start 134.59 79.344999) (end 134.59 78.49) (width 0.25) (layer F.Cu) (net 8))
 (segment (start 135.09 80.495) (end 135.09 81.39) (width 0.25) (layer F.Cu) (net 5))
 (segment (start 135.1 83.53) (end 135.1 81.46) (width 0.5) (layer F.Cu) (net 5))
 (segment (start 135.395 83.825) (end 135.1 83.53) (width 0.5) (layer F.Cu) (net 5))
 (segment (start 137.935 83.825) (end 135.395 83.825) (width 0.5) (layer F.Cu) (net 5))
 (segment (start 136.385 80.495) (end 136.46 80.42) (width 0.5) (layer F.Cu) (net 2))
 (segment (start 135.71 80.5) (end 136.505 80.5) (width 0.5) (layer F.Cu) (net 2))
 (segment (start 136.555 80.515) (end 137.935 80.515) (width 0.5) (layer F.Cu) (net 2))
 (segment (start 136.46 80.42) (end 136.555 80.515) (width 0.5) (layer F.Cu) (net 2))
 (segment (start 140.805 80.515) (end 140.804999 78.565) (width 0.5) (layer F.Cu) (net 4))
 (segment (start 140.805 83.825) (end 140.805 81.875) (width 0.5) (layer F.Cu) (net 4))
 (segment (start 140.805 80.515) (end 140.805 81.875) (width 0.5) (layer F.Cu) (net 4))
 (segment (start 140.58001 82.30001) (end 140.805 82.525) (width 0.5) (layer F.Cu) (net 4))
 (segment (start 140.58001 80.201468) (end 140.58001 82.30001) (width 0.5) (layer F.Cu) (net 4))
 (segment (start 140.805 80.426458) (end 140.58001 80.201468) (width 0.5) (layer F.Cu) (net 4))
 (segment (start 140.805 80.515) (end 140.805 80.426458) (width 0.5) (layer F.Cu) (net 4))
 (segment (start 140.47 80.515) (end 140.47 81.875) (width 0.5) (layer F.Cu) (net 4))
 (segment (start 125.34 78.91) (end 125.33 78.92) (width 0.5) (layer F.Cu) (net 1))
 (segment (start 126.7 78.910001) (end 125.34 78.91) (width 0.5) (layer F.Cu) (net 1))
 (segment (start 137.935 83.175) (end 137.934999 81.875) (width 0.5) (layer F.Cu) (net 1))
 (via (at 136.07 81.92) (size 0.4) (drill 0.3) (layers F.Cu B.Cu) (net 1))
 (via (at 136.07 82.66) (size 0.4) (drill 0.3) (layers F.Cu B.Cu) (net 1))
 (via (at 136.82 81.92) (size 0.4) (drill 0.3) (layers F.Cu B.Cu) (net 1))
 (via (at 136.82 82.66) (size 0.4) (drill 0.3) (layers F.Cu B.Cu) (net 1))
 (via (at 124.44 84.7) (size 0.4) (drill 0.3) (layers F.Cu B.Cu) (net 1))
 (via (at 124.44 83.96) (size 0.4) (drill 0.3) (layers F.Cu B.Cu) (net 1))
 (via (at 125.25 84.7) (size 0.4) (drill 0.3) (layers F.Cu B.Cu) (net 1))
 (via (at 126 83.96) (size 0.4) (drill 0.3) (layers F.Cu B.Cu) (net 1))
 (via (at 126 84.7) (size 0.4) (drill 0.3) (layers F.Cu B.Cu) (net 1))
 (via (at 125.25 83.96) (size 0.4) (drill 0.3) (layers F.Cu B.Cu) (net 1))
 (via (at 127.85 84.7) (size 0.4) (drill 0.3) (layers F.Cu B.Cu) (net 1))
 (via (at 127.1 84.7) (size 0.4) (drill 0.3) (layers F.Cu B.Cu) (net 1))
 (via (at 127.85 83.96) (size 0.4) (drill 0.3) (layers F.Cu B.Cu) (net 1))
 (via (at 127.1 83.96) (size 0.4) (drill 0.3) (layers F.Cu B.Cu) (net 1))
 (via (at 126 83.23) (size 0.4) (drill 0.3) (layers F.Cu B.Cu) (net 1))
 (via (at 124.44 83.23) (size 0.4) (drill 0.3) (layers F.Cu B.Cu) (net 1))
 (via (at 125.25 83.23) (size 0.4) (drill 0.3) (layers F.Cu B.Cu) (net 1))
 (via (at 127.85 83.23) (size 0.4) (drill 0.3) (layers F.Cu B.Cu) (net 1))
 (via (at 127.1 83.23) (size 0.4) (drill 0.3) (layers F.Cu B.Cu) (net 1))
 (via (at 125.32 79.809999) (size 0.4) (drill 0.3) (layers F.Cu B.Cu) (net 1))
 (via (at 124.57 79.81) (size 0.4) (drill 0.3) (layers F.Cu B.Cu) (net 1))
 (via (at 124.18 76.87) (size 0.4) (drill 0.3) (layers F.Cu B.Cu) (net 1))
 (via (at 124.93 76.869999) (size 0.4) (drill 0.3) (layers F.Cu B.Cu) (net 1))
 (via (at 124.93 76.099999) (size 0.4) (drill 0.3) (layers F.Cu B.Cu) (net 1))
 (via (at 124.18 76.1) (size 0.4) (drill 0.3) (layers F.Cu B.Cu) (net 1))
 (via (at 126.51 76.869999) (size 0.4) (drill 0.3) (layers F.Cu B.Cu) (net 1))
 (via (at 125.76 76.1) (size 0.4) (drill 0.3) (layers F.Cu B.Cu) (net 1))
 (via (at 125.76 76.87) (size 0.4) (drill 0.3) (layers F.Cu B.Cu) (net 1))
 (via (at 126.51 76.099999) (size 0.4) (drill 0.3) (layers F.Cu B.Cu) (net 1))
 (via (at 132.32 80.139999) (size 0.4) (drill 0.3) (layers F.Cu B.Cu) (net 1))
 (via (at 131.57 80.91) (size 0.4) (drill 0.3) (layers F.Cu B.Cu) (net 1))
 (via (at 132.32 80.909999) (size 0.4) (drill 0.3) (layers F.Cu B.Cu) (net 1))
 (via (at 131.57 80.14) (size 0.4) (drill 0.3) (layers F.Cu B.Cu) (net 1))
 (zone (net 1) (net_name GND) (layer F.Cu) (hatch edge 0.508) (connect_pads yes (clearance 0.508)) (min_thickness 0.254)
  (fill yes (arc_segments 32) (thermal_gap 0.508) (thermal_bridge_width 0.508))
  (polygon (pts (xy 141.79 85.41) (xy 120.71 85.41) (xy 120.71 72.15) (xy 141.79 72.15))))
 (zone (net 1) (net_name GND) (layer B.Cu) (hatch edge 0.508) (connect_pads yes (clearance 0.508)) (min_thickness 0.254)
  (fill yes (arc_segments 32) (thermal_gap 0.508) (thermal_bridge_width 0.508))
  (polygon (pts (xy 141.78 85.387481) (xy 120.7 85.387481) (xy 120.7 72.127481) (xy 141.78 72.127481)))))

